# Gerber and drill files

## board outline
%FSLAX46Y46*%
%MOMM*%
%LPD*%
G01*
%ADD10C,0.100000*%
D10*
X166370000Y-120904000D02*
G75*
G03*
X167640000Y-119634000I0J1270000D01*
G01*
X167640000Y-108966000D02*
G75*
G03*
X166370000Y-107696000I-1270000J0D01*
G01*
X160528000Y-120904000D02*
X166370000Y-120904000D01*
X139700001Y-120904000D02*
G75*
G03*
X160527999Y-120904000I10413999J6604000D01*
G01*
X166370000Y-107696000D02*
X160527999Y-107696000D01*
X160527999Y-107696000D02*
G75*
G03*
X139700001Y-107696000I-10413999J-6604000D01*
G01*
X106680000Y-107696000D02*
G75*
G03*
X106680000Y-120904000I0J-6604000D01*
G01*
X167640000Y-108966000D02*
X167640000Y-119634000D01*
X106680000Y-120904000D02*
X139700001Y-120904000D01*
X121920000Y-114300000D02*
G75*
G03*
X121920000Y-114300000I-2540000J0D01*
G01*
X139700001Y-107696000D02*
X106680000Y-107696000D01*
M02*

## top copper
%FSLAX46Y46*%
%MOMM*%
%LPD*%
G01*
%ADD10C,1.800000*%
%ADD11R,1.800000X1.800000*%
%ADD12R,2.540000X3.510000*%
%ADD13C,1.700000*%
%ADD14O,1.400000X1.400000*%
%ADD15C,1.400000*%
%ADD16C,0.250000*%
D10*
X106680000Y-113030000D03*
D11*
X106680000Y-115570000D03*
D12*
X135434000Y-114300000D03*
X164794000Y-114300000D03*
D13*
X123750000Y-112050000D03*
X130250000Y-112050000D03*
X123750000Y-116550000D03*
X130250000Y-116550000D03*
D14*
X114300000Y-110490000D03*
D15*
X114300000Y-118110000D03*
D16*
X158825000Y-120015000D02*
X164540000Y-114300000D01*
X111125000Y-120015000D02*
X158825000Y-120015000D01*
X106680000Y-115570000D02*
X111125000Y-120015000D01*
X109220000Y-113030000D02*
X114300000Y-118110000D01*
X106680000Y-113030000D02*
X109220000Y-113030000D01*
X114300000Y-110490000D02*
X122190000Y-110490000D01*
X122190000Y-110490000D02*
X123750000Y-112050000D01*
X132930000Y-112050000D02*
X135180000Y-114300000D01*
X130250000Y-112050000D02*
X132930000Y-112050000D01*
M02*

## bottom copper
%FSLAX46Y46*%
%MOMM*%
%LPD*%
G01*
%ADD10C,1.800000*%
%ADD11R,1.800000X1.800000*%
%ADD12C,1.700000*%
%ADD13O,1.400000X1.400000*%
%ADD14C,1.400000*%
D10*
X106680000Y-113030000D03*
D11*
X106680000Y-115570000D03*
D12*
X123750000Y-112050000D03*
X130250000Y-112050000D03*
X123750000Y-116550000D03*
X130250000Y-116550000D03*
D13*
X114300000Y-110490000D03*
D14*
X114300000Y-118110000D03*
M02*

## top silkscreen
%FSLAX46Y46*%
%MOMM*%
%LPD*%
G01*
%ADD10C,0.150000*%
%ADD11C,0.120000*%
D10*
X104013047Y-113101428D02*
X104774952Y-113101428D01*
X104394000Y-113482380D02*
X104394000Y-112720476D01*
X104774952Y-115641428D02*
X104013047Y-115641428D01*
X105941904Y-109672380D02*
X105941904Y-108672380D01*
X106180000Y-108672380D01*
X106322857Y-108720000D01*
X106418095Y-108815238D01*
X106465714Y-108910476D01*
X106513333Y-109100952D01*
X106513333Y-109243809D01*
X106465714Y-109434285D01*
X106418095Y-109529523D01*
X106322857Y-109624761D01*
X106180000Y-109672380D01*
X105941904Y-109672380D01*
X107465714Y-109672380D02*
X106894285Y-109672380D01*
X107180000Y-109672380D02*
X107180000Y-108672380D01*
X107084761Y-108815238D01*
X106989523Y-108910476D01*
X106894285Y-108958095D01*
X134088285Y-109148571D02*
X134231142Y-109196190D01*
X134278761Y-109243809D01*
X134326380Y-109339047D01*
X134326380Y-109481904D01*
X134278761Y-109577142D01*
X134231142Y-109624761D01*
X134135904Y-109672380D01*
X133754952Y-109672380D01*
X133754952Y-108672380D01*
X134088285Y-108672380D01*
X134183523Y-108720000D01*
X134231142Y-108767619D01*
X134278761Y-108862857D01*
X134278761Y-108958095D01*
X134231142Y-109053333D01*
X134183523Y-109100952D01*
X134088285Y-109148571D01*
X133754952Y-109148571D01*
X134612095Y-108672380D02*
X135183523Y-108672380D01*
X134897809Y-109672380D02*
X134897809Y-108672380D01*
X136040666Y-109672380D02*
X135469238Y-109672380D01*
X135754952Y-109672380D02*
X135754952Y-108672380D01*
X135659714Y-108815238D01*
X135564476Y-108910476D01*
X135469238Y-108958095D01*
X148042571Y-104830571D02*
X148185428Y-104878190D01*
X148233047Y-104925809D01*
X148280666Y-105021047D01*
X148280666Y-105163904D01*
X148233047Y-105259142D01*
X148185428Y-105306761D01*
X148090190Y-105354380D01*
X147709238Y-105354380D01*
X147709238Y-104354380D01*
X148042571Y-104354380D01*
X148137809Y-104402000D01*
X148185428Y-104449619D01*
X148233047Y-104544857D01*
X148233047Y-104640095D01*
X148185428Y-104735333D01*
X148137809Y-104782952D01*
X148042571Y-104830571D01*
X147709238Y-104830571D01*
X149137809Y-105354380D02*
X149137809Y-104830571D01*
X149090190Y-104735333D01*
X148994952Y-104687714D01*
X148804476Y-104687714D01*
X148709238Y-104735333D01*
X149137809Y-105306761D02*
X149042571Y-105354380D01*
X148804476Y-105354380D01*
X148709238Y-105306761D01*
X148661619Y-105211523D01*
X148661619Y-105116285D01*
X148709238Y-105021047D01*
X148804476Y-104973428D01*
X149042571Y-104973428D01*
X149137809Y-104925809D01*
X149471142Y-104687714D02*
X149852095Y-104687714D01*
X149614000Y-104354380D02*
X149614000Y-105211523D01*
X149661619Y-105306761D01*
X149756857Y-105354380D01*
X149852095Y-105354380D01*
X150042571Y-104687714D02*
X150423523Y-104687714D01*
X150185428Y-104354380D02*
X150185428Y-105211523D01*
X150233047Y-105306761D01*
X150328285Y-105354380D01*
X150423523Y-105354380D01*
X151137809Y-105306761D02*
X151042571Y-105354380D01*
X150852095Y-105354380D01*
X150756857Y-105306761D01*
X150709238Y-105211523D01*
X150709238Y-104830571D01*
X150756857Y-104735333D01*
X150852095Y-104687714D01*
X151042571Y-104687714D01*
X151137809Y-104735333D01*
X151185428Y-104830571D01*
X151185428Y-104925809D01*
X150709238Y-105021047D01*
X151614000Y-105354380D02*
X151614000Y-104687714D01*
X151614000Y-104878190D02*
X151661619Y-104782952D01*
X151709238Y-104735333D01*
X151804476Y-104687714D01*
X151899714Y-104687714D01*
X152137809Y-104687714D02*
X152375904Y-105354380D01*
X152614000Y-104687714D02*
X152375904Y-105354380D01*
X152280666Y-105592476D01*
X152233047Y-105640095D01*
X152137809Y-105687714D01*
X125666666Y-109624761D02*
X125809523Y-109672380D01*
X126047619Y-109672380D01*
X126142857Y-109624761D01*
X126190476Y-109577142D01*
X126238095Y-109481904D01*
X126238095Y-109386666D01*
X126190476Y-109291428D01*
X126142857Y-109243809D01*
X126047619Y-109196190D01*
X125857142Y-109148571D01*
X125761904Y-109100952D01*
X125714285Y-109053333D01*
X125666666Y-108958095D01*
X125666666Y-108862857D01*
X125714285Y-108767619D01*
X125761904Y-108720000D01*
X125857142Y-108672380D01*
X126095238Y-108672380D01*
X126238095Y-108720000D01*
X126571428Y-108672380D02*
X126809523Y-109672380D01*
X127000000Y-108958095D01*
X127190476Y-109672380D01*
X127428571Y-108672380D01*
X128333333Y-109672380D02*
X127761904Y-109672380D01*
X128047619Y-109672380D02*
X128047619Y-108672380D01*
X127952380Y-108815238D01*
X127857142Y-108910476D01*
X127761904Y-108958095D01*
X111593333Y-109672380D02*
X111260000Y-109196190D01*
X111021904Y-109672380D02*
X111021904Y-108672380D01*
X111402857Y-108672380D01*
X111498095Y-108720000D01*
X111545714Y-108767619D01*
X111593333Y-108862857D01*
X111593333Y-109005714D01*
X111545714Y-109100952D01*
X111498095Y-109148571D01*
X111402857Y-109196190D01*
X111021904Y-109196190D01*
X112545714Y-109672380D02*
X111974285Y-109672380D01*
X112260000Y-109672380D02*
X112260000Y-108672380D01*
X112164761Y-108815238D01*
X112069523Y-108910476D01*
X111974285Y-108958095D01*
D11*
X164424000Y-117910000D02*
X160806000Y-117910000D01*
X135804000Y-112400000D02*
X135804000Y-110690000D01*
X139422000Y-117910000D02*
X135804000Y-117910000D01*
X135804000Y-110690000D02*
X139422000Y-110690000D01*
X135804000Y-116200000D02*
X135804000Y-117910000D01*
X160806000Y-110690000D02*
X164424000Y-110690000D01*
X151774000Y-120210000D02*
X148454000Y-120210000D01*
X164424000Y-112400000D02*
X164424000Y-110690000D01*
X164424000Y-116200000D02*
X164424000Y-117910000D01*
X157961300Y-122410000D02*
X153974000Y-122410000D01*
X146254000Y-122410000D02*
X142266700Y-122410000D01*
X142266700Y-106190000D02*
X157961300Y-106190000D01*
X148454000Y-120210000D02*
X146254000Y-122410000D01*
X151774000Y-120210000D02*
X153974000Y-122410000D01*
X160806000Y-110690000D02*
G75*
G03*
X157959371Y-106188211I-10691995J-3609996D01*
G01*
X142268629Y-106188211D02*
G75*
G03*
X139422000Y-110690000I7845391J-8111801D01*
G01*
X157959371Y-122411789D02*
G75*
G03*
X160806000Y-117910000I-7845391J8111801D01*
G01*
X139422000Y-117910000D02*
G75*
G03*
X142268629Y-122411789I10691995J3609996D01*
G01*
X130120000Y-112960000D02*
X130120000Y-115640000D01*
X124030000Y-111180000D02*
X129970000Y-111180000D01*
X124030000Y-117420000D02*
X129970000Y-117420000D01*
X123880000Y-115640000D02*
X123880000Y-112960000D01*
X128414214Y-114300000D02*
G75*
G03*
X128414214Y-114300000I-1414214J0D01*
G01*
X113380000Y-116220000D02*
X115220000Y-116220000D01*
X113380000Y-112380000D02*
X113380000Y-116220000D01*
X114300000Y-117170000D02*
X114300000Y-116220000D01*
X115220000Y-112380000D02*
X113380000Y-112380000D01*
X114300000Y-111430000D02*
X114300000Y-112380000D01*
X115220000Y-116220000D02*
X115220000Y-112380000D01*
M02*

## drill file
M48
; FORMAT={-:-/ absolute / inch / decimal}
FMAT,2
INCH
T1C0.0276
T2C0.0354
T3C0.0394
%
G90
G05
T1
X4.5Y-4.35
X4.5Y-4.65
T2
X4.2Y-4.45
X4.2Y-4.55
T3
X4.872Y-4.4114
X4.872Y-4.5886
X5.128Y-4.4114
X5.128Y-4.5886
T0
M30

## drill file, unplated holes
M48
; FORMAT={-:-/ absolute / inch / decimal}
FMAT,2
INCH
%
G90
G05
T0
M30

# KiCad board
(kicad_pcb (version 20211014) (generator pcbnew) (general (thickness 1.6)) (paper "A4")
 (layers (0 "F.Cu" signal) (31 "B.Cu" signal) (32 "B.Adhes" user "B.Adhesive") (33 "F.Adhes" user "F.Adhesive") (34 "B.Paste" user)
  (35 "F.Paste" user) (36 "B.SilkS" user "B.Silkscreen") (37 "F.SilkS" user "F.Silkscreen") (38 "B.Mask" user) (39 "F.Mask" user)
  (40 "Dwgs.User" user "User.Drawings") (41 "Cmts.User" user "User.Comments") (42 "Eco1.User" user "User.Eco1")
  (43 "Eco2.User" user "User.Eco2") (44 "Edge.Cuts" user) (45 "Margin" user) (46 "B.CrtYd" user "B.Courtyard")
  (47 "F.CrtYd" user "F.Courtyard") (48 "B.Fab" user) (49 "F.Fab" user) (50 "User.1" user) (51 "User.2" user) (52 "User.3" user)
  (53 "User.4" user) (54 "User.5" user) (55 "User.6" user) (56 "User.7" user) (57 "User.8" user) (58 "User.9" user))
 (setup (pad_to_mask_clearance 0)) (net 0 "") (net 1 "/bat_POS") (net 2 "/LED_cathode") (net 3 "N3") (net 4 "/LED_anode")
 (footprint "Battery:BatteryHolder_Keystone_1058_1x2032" (layer "F.Cu") (at 150.114 114.3)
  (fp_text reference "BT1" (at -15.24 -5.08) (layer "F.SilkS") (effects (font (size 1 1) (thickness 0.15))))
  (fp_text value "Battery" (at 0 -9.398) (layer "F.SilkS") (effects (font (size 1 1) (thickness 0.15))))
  (fp_line (start 14.31 3.61) (end 10.692 3.61) (layer "F.SilkS") (width 0.12))
  (fp_line (start -14.31 -1.9) (end -14.31 -3.61) (layer "F.SilkS") (width 0.12))
  (fp_line (start -10.692 3.61) (end -14.31 3.61) (layer "F.SilkS") (width 0.12))
  (fp_line (start -14.31 -3.61) (end -10.692 -3.61) (layer "F.SilkS") (width 0.12))
  (fp_line (start -14.31 1.9) (end -14.31 3.61) (layer "F.SilkS") (width 0.12))
  (fp_line (start 10.692 -3.61) (end 14.31 -3.61) (layer "F.SilkS") (width 0.12))
  (fp_line (start 1.66 5.91) (end -1.66 5.91) (layer "F.SilkS") (width 0.12))
  (fp_line (start 14.31 -1.9) (end 14.31 -3.61) (layer "F.SilkS") (width 0.12))
  (fp_line (start 14.31 1.9) (end 14.31 3.61) (layer "F.SilkS") (width 0.12))
  (fp_line (start 7.8473 8.11) (end 3.86 8.11) (layer "F.SilkS") (width 0.12))
  (fp_line (start -3.86 8.11) (end -7.8473 8.11) (layer "F.SilkS") (width 0.12))
  (fp_line (start -7.8473 -8.11) (end 7.8473 -8.11) (layer "F.SilkS") (width 0.12))
  (fp_line (start -1.66 5.91) (end -3.86 8.11) (layer "F.SilkS") (width 0.12))
  (fp_line (start 1.66 5.91) (end 3.86 8.11) (layer "F.SilkS") (width 0.12))
  (fp_arc (start 7.845371 -8.111789) (mid 9.538085 -6.031244) (end 10.692 -3.61) (layer "F.SilkS") (width 0.12))
  (fp_arc (start -10.692 -3.61) (mid -9.538084 -6.031244) (end -7.845371 -8.111789) (layer "F.SilkS") (width 0.12))
  (fp_arc (start 10.692 3.61) (mid 9.538084 6.031244) (end 7.845371 8.111789) (layer "F.SilkS") (width 0.12))
  (fp_arc (start -7.845371 8.111789) (mid -9.538085 6.031244) (end -10.692 3.61) (layer "F.SilkS") (width 0.12))
  (pad "1" smd rect locked (at -14.68 0) (size 2.54 3.51) (layers "F.Cu" "F.Paste" "F.Mask") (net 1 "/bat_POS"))
  (pad "2" smd rect locked (at 14.68 0) (size 2.54 3.51) (layers "F.Cu" "F.Paste" "F.Mask") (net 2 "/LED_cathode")))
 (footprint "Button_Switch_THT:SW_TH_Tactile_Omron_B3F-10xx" (layer "F.Cu") (at 123.75 112.05)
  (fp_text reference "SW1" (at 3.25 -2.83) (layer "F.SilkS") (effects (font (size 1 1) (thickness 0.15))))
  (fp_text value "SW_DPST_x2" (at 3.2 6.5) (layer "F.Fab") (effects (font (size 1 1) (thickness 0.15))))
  (fp_line (start 6.37 0.91) (end 6.37 3.59) (layer "F.SilkS") (width 0.12))
  (fp_line (start 0.28 -0.87) (end 6.22 -0.87) (layer "F.SilkS") (width 0.12))
  (fp_line (start 0.28 5.37) (end 6.22 5.37) (layer "F.SilkS") (width 0.12))
  (fp_line (start 0.13 3.59) (end 0.13 0.91) (layer "F.SilkS") (width 0.12))
  (fp_circle (center 3.25 2.25) (end 4.25 3.25) (layer "F.SilkS") (width 0.12) (fill none))
  (pad "1" thru_hole circle locked (at 0 0) (size 1.7 1.7) (drill 1) (layers *.Cu *.Mask) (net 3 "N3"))
  (pad "2" thru_hole circle locked (at 6.5 0) (size 1.7 1.7) (drill 1) (layers *.Cu *.Mask) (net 1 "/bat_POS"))
  (pad "3" thru_hole circle locked (at 0 4.5) (size 1.7 1.7) (drill 1) (layers *.Cu *.Mask))
  (pad "4" thru_hole circle locked (at 6.5 4.5) (size 1.7 1.7) (drill 1) (layers *.Cu *.Mask)))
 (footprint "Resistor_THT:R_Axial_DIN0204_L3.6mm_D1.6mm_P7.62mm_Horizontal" (layer "F.Cu") (at 114.3 118.11 90)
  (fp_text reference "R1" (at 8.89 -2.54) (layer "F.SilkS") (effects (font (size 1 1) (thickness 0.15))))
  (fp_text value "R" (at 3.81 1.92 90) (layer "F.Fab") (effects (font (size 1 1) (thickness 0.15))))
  (fp_line (start 1.89 0.92) (end 5.73 0.92) (layer "F.SilkS") (width 0.12))
  (fp_line (start 6.68 0) (end 5.73 0) (layer "F.SilkS") (width 0.12))
  (fp_line (start 5.73 0.92) (end 5.73 -0.92) (layer "F.SilkS") (width 0.12))
  (fp_line (start 0.94 0) (end 1.89 0) (layer "F.SilkS") (width 0.12))
  (fp_line (start 5.73 -0.92) (end 1.89 -0.92) (layer "F.SilkS") (width 0.12))
  (fp_line (start 1.89 -0.92) (end 1.89 0.92) (layer "F.SilkS") (width 0.12))
  (pad "1" thru_hole circle locked (at 0 0 90) (size 1.4 1.4) (drill 0.7) (layers *.Cu *.Mask) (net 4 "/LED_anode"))
  (pad "2" thru_hole oval locked (at 7.62 0 90) (size 1.4 1.4) (drill 0.7) (layers *.Cu *.Mask) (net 3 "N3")))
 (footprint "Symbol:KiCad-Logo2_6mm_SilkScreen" (layer "B.Cu") (at 150.114 114.3 180)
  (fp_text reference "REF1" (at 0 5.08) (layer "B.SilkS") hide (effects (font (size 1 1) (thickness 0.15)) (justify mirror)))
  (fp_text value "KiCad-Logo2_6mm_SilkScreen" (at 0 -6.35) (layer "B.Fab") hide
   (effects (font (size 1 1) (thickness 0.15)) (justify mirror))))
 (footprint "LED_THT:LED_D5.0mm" (layer "B.Cu") (at 106.68 115.57 90)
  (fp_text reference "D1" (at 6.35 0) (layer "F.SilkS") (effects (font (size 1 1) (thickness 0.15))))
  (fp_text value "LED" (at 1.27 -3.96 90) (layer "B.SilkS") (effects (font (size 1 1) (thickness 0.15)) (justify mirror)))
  (pad "1" thru_hole rect locked (at 0 0 90) (size 1.8 1.8) (drill 0.9) (layers *.Cu *.Mask) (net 2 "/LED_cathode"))
  (pad "2" thru_hole circle locked (at 2.54 0 90) (size 1.8 1.8) (drill 0.9) (layers *.Cu *.Mask) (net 4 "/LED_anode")))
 (gr_arc (start 160.527999 120.904) (mid 150.114 126.631431) (end 139.700001 120.904) (layer "Edge.Cuts") (width 0.1))
 (gr_line (start 166.37 107.696) (end 160.527999 107.696) (layer "Edge.Cuts") (width 0.1))
 (gr_line (start 160.528 120.904) (end 166.37 120.904) (layer "Edge.Cuts") (width 0.1))
 (gr_arc (start 139.700001 107.696) (mid 150.114 101.968569) (end 160.527999 107.696) (layer "Edge.Cuts") (width 0.1))
 (gr_arc (start 167.64 119.634) (mid 167.268026 120.532026) (end 166.37 120.904) (layer "Edge.Cuts") (width 0.1))
 (gr_line (start 106.68 120.904) (end 139.700001 120.904) (layer "Edge.Cuts") (width 0.1))
 (gr_arc (start 166.37 107.696) (mid 167.268026 108.067974) (end 167.64 108.966) (layer "Edge.Cuts") (width 0.1))
 (gr_circle (center 119.38 114.3) (end 121.92 114.3) (layer "Edge.Cuts") (width 0.1) (fill none))
 (gr_arc (start 106.68 120.904) (mid 100.076 114.3) (end 106.68 107.696) (layer "Edge.Cuts") (width 0.1))
 (gr_line (start 139.700001 107.696) (end 106.68 107.696) (layer "Edge.Cuts") (width 0.1))
 (gr_line (start 167.64 108.966) (end 167.64 119.634) (layer "Edge.Cuts") (width 0.1))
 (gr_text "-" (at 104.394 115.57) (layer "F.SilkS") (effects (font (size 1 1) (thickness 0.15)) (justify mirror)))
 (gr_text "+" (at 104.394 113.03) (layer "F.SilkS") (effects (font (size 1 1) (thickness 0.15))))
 (segment (start 132.93 112.05) (end 135.18 114.3) (width 0.25) (layer "F.Cu") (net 1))
 (segment (start 130.25 112.05) (end 132.93 112.05) (width 0.25) (layer "F.Cu") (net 1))
 (segment (start 158.825 120.015) (end 164.54 114.3) (width 0.25) (layer "F.Cu") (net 2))
 (segment (start 111.125 120.015) (end 158.825 120.015) (width 0.25) (layer "F.Cu") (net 2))
 (segment (start 106.68 115.57) (end 111.125 120.015) (width 0.25) (layer "F.Cu") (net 2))
 (segment (start 106.68 113.03) (end 109.22 113.03) (width 0.25) (layer "F.Cu") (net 4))
 (segment (start 109.22 113.03) (end 114.3 118.11) (width 0.25) (layer "F.Cu") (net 4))
 (segment (start 114.3 110.49) (end 122.19 110.49) (width 0.25) (layer "F.Cu") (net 3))
 (segment (start 122.19 110.49) (end 123.75 112.05) (width 0.25) (layer "F.Cu") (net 3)))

